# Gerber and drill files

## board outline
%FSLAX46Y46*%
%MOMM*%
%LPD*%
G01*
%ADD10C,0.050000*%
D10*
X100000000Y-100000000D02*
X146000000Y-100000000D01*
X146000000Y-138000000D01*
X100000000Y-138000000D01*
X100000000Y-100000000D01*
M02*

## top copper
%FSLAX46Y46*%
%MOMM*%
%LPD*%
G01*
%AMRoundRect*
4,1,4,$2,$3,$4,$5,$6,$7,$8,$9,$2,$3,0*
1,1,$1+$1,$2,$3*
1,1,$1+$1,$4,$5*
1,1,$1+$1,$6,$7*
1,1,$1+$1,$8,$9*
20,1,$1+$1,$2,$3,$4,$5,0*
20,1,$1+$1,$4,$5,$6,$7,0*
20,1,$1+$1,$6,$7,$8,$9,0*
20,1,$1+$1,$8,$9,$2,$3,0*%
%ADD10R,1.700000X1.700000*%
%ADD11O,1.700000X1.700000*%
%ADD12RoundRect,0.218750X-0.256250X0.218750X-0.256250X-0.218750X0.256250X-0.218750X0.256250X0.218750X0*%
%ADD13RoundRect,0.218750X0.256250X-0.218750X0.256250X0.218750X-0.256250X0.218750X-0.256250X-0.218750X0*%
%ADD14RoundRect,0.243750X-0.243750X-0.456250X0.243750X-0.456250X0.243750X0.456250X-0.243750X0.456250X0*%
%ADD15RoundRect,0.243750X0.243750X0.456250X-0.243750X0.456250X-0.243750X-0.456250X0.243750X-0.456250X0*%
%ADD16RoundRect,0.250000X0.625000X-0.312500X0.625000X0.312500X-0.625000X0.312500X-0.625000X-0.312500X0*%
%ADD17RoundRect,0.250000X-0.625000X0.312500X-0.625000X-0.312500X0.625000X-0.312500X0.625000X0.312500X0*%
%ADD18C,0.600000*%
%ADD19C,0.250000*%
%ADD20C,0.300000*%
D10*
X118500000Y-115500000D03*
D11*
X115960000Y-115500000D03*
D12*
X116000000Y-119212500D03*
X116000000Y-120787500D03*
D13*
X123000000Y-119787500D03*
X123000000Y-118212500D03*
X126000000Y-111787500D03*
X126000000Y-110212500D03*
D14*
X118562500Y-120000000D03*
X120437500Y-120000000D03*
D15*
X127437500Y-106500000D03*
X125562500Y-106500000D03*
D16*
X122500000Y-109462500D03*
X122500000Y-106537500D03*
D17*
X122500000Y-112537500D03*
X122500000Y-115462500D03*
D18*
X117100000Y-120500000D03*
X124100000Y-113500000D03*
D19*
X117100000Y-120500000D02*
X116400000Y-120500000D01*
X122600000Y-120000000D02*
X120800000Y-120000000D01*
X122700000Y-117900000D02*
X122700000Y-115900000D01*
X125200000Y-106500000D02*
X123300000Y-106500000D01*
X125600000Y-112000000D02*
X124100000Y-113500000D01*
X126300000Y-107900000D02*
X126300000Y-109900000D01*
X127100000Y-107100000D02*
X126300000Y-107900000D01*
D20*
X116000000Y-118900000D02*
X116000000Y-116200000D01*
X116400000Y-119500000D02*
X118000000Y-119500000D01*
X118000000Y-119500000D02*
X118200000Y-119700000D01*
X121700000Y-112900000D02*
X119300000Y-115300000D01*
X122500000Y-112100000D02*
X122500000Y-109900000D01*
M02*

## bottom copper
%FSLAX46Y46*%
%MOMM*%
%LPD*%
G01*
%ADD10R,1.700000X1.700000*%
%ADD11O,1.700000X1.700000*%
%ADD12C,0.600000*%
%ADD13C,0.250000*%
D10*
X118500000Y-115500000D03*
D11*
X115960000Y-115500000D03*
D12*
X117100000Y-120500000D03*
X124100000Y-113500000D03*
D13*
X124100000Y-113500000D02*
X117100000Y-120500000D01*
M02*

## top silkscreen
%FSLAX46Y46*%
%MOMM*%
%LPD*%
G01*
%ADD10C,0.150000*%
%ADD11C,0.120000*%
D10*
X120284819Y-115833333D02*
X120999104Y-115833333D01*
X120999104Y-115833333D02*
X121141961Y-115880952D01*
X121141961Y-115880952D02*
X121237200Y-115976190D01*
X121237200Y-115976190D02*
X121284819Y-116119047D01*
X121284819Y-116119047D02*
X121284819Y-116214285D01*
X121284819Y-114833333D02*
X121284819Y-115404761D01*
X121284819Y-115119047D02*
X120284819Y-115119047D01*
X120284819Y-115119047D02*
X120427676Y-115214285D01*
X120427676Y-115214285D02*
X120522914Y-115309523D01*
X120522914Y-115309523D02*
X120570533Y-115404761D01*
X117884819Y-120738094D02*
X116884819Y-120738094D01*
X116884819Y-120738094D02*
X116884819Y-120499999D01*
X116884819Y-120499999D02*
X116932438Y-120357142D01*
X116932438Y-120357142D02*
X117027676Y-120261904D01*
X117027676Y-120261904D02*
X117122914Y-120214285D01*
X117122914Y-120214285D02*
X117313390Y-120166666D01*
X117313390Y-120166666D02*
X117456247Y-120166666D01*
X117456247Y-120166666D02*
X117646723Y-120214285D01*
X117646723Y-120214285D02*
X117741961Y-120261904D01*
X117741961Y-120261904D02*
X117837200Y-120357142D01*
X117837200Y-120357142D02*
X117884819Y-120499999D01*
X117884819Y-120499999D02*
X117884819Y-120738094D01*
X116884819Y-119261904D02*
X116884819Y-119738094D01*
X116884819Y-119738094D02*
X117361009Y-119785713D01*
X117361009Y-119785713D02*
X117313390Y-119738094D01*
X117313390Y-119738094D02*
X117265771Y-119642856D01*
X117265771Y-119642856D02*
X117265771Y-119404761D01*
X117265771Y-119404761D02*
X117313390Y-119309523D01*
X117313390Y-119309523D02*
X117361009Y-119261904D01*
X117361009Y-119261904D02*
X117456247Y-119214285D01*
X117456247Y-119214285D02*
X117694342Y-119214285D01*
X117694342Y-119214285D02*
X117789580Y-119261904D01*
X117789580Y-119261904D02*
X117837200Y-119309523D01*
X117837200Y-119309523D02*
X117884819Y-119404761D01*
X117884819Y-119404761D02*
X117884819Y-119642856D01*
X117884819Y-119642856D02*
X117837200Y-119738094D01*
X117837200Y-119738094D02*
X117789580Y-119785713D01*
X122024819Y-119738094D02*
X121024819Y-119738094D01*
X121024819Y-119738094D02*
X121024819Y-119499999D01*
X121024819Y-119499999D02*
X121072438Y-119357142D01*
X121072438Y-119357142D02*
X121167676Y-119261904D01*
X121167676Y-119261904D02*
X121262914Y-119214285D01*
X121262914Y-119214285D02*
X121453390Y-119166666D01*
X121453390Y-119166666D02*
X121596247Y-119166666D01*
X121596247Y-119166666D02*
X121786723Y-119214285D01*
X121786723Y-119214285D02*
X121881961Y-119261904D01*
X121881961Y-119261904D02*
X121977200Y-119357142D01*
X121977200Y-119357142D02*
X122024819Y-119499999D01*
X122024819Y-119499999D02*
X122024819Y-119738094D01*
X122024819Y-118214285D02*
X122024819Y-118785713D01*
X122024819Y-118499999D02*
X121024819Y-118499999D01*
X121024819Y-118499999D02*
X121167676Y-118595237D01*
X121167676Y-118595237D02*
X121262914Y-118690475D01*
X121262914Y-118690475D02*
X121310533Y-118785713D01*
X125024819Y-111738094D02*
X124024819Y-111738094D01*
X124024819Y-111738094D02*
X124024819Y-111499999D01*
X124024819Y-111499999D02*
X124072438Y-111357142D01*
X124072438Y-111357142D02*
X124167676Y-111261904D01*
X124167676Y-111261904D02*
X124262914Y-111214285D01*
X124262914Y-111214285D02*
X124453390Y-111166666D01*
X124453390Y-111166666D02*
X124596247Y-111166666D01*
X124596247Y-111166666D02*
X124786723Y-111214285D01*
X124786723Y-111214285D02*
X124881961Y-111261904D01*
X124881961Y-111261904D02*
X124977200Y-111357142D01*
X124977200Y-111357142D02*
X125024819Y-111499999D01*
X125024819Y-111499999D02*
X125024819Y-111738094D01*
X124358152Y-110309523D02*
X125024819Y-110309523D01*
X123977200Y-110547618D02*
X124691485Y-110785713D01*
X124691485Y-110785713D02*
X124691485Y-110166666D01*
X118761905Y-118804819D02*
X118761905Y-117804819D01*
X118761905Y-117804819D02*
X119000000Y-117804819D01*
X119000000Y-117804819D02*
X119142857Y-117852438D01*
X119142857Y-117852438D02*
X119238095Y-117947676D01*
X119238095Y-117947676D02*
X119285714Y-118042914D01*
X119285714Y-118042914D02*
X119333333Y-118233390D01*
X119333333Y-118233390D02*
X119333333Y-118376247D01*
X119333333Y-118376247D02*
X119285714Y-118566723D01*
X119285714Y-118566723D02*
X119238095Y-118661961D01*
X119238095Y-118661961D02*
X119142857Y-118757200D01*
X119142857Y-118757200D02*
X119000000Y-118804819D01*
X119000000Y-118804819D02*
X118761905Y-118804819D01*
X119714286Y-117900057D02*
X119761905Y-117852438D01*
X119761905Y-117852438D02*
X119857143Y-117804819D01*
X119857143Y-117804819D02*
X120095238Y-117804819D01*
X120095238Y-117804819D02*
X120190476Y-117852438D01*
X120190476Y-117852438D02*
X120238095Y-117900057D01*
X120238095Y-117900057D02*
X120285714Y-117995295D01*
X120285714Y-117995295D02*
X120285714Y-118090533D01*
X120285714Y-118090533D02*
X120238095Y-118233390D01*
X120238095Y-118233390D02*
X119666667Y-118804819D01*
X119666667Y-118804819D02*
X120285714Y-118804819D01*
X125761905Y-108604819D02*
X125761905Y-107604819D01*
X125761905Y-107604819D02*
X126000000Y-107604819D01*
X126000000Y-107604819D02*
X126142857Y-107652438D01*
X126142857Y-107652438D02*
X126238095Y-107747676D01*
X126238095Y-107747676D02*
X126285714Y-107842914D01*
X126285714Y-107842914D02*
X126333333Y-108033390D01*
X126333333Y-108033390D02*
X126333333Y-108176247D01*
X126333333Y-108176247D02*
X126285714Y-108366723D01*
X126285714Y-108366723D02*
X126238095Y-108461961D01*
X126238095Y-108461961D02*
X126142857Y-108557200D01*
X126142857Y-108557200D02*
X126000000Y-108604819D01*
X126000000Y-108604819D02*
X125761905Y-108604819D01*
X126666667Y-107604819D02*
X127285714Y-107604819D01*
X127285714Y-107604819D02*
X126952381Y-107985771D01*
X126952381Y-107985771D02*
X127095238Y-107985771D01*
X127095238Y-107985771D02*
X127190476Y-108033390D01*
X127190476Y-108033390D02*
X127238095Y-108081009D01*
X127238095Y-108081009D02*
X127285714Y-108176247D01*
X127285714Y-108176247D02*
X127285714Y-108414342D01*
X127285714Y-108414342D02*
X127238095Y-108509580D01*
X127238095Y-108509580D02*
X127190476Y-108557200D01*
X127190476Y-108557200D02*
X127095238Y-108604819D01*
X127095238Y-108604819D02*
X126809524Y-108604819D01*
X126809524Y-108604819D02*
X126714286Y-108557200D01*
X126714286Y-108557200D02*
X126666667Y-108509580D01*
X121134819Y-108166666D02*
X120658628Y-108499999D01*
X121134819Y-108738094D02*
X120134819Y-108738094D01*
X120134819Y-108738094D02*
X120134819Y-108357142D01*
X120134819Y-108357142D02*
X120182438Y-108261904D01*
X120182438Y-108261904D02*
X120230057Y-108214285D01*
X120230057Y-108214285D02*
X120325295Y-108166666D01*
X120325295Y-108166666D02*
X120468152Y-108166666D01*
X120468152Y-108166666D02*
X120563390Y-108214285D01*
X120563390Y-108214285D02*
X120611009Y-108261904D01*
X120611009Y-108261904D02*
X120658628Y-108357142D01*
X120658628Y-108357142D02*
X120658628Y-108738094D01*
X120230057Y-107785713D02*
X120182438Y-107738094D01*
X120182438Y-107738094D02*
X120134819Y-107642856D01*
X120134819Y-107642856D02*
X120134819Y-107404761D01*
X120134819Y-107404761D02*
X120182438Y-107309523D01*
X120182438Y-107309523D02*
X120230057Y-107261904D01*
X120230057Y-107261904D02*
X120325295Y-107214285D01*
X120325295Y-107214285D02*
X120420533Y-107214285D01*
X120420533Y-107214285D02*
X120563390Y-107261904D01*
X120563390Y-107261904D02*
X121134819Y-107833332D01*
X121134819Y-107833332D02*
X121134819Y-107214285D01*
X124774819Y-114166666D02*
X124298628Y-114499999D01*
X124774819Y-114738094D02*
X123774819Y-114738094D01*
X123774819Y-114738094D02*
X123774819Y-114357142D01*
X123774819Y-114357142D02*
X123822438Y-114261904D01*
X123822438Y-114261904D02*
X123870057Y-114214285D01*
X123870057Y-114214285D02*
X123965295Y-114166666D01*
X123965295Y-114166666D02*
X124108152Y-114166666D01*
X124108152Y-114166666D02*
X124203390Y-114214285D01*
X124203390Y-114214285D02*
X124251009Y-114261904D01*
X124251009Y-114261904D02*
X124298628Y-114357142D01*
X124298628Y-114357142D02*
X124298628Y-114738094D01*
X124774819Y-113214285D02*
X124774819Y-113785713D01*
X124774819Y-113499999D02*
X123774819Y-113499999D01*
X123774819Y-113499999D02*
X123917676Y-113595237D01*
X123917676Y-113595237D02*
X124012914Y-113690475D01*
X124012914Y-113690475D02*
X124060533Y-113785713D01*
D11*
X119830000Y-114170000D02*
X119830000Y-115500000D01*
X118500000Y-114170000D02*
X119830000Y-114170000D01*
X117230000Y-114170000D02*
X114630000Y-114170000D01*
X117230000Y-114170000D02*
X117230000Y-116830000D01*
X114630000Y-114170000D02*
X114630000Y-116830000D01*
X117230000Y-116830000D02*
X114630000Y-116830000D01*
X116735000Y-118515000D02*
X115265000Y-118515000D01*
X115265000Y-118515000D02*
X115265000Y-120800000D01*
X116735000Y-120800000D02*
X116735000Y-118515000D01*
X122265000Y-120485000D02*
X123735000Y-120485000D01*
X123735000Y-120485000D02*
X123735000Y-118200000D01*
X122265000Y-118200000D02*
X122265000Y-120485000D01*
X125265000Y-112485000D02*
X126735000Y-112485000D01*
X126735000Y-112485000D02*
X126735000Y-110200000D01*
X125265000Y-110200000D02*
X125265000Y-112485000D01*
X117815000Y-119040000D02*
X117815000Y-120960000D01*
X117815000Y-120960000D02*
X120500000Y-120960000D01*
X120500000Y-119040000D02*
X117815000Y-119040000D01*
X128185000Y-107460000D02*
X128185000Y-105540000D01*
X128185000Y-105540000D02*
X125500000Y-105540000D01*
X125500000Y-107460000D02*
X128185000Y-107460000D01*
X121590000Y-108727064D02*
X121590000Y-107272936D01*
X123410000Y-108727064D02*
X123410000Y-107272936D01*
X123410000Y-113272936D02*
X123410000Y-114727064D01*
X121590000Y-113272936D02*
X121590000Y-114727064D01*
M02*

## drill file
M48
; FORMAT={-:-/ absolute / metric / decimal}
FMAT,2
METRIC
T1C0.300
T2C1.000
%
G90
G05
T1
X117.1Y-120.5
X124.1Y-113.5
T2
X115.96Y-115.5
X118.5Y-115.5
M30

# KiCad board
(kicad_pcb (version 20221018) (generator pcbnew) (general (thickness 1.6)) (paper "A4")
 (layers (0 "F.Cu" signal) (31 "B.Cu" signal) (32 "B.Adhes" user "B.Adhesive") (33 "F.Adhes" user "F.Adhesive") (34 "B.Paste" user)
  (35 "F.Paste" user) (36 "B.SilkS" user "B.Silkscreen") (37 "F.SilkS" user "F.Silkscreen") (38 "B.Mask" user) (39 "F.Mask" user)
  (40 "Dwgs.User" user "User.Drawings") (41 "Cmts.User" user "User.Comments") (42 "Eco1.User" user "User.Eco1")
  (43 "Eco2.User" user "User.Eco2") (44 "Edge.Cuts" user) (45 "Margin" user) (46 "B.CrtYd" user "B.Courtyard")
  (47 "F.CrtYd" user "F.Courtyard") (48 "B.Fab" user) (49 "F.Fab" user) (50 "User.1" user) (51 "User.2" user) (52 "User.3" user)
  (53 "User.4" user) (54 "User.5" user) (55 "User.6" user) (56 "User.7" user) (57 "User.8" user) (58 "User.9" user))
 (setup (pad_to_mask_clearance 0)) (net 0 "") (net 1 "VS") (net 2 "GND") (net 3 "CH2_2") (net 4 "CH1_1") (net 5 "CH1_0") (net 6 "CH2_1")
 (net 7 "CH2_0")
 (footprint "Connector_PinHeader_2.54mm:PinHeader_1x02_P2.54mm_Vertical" (layer "F.Cu") (at 118.5 115.5 -90)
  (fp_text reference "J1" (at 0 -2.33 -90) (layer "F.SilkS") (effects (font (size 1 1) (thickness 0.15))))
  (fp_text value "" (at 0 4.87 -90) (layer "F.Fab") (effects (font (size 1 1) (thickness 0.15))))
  (fp_line (start -1.33 -1.33) (end 0 -1.33) (stroke (width 0.12) (type solid)) (layer "F.SilkS"))
  (fp_line (start -1.33 0) (end -1.33 -1.33) (stroke (width 0.12) (type solid)) (layer "F.SilkS"))
  (fp_line (start -1.33 1.27) (end -1.33 3.87) (stroke (width 0.12) (type solid)) (layer "F.SilkS"))
  (fp_line (start -1.33 1.27) (end 1.33 1.27) (stroke (width 0.12) (type solid)) (layer "F.SilkS"))
  (fp_line (start -1.33 3.87) (end 1.33 3.87) (stroke (width 0.12) (type solid)) (layer "F.SilkS"))
  (fp_line (start 1.33 1.27) (end 1.33 3.87) (stroke (width 0.12) (type solid)) (layer "F.SilkS"))
  (pad "1" thru_hole rect (at 0 0 270) (size 1.7 1.7) (drill 1) (layers "*.Cu" "*.Mask") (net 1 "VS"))
  (pad "2" thru_hole oval (at 0 2.54 270) (size 1.7 1.7) (drill 1) (layers "*.Cu" "*.Mask") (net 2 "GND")))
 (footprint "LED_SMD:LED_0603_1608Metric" (layer "F.Cu") (at 116 120 -90)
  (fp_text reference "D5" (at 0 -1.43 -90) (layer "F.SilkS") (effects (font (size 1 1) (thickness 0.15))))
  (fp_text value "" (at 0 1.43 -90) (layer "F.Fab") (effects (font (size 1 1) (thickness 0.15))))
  (fp_line (start -1.485 -0.735) (end -1.485 0.735) (stroke (width 0.12) (type solid)) (layer "F.SilkS"))
  (fp_line (start -1.485 0.735) (end 0.8 0.735) (stroke (width 0.12) (type solid)) (layer "F.SilkS"))
  (fp_line (start 0.8 -0.735) (end -1.485 -0.735) (stroke (width 0.12) (type solid)) (layer "F.SilkS"))
  (pad "1" smd roundrect (at -0.7875 0 270) (size 0.875 0.95) (layers "F.Cu" "F.Paste" "F.Mask") (roundrect_rratio 0.25) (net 2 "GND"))
  (pad "2" smd roundrect (at 0.7875 0 270) (size 0.875 0.95) (layers "F.Cu" "F.Paste" "F.Mask") (roundrect_rratio 0.25) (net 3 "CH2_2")))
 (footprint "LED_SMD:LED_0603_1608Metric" (layer "F.Cu") (at 123 119 90)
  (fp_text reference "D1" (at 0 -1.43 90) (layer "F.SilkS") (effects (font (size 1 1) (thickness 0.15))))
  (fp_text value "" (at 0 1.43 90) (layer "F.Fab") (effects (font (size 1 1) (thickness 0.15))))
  (fp_line (start -1.485 -0.735) (end -1.485 0.735) (stroke (width 0.12) (type solid)) (layer "F.SilkS"))
  (fp_line (start -1.485 0.735) (end 0.8 0.735) (stroke (width 0.12) (type solid)) (layer "F.SilkS"))
  (fp_line (start 0.8 -0.735) (end -1.485 -0.735) (stroke (width 0.12) (type solid)) (layer "F.SilkS"))
  (pad "1" smd roundrect (at -0.7875 0 90) (size 0.875 0.95) (layers "F.Cu" "F.Paste" "F.Mask") (roundrect_rratio 0.25) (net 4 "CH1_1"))
  (pad "2" smd roundrect (at 0.7875 0 90) (size 0.875 0.95) (layers "F.Cu" "F.Paste" "F.Mask") (roundrect_rratio 0.25) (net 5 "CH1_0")))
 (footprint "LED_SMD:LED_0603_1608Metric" (layer "F.Cu") (at 126 111 90)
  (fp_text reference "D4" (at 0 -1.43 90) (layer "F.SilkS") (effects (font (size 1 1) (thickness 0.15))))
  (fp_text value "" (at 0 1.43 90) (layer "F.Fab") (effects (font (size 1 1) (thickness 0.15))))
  (fp_line (start -1.485 -0.735) (end -1.485 0.735) (stroke (width 0.12) (type solid)) (layer "F.SilkS"))
  (fp_line (start -1.485 0.735) (end 0.8 0.735) (stroke (width 0.12) (type solid)) (layer "F.SilkS"))
  (fp_line (start 0.8 -0.735) (end -1.485 -0.735) (stroke (width 0.12) (type solid)) (layer "F.SilkS"))
  (pad "1" smd roundrect (at -0.7875 0 90) (size 0.875 0.95) (layers "F.Cu" "F.Paste" "F.Mask") (roundrect_rratio 0.25) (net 3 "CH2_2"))
  (pad "2" smd roundrect (at 0.7875 0 90) (size 0.875 0.95) (layers "F.Cu" "F.Paste" "F.Mask") (roundrect_rratio 0.25) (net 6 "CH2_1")))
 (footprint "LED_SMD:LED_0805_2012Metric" (layer "F.Cu") (at 119.5 120)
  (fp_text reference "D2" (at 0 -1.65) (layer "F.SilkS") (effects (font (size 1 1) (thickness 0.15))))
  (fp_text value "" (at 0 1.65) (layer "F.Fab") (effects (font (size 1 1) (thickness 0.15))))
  (fp_line (start -1.685 -0.96) (end -1.685 0.96) (stroke (width 0.12) (type solid)) (layer "F.SilkS"))
  (fp_line (start -1.685 0.96) (end 1 0.96) (stroke (width 0.12) (type solid)) (layer "F.SilkS"))
  (fp_line (start 1 -0.96) (end -1.685 -0.96) (stroke (width 0.12) (type solid)) (layer "F.SilkS"))
  (pad "1" smd roundrect (at -0.9375 0) (size 0.975 1.4) (layers "F.Cu" "F.Paste" "F.Mask") (roundrect_rratio 0.25) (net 2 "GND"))
  (pad "2" smd roundrect (at 0.9375 0) (size 0.975 1.4) (layers "F.Cu" "F.Paste" "F.Mask") (roundrect_rratio 0.25) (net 4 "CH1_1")))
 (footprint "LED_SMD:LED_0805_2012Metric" (layer "F.Cu") (at 126.5 106.5 180)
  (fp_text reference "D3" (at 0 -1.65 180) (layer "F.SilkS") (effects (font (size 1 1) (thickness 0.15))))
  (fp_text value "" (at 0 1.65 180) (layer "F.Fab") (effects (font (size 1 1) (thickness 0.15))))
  (fp_line (start -1.685 -0.96) (end -1.685 0.96) (stroke (width 0.12) (type solid)) (layer "F.SilkS"))
  (fp_line (start -1.685 0.96) (end 1 0.96) (stroke (width 0.12) (type solid)) (layer "F.SilkS"))
  (fp_line (start 1 -0.96) (end -1.685 -0.96) (stroke (width 0.12) (type solid)) (layer "F.SilkS"))
  (pad "1" smd roundrect (at -0.9375 0 180) (size 0.975 1.4) (layers "F.Cu" "F.Paste" "F.Mask") (roundrect_rratio 0.25) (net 6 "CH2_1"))
  (pad "2" smd roundrect (at 0.9375 0 180) (size 0.975 1.4) (layers "F.Cu" "F.Paste" "F.Mask") (roundrect_rratio 0.25) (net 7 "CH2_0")))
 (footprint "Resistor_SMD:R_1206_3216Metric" (layer "F.Cu") (at 122.5 108 90)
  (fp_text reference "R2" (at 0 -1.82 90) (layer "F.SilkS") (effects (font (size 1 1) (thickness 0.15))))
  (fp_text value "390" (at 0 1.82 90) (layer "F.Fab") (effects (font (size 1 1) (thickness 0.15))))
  (fp_line (start -0.727064 -0.91) (end 0.727064 -0.91) (stroke (width 0.12) (type solid)) (layer "F.SilkS"))
  (fp_line (start -0.727064 0.91) (end 0.727064 0.91) (stroke (width 0.12) (type solid)) (layer "F.SilkS"))
  (pad "1" smd roundrect (at -1.4625 0 90) (size 1.125 1.75) (layers "F.Cu" "F.Paste" "F.Mask") (roundrect_rratio 0.222222) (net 1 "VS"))
  (pad "2" smd roundrect (at 1.4625 0 90) (size 1.125 1.75) (layers "F.Cu" "F.Paste" "F.Mask") (roundrect_rratio 0.222222) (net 7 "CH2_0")))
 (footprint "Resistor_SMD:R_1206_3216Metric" (layer "F.Cu") (at 122.5 114 -90)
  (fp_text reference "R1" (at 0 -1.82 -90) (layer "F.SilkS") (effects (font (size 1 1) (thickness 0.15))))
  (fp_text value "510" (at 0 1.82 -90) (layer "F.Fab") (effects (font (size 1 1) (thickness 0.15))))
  (fp_line (start -0.727064 -0.91) (end 0.727064 -0.91) (stroke (width 0.12) (type solid)) (layer "F.SilkS"))
  (fp_line (start -0.727064 0.91) (end 0.727064 0.91) (stroke (width 0.12) (type solid)) (layer "F.SilkS"))
  (pad "1" smd roundrect (at -1.4625 0 270) (size 1.125 1.75) (layers "F.Cu" "F.Paste" "F.Mask") (roundrect_rratio 0.222222) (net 1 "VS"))
  (pad "2" smd roundrect (at 1.4625 0 270) (size 1.125 1.75) (layers "F.Cu" "F.Paste" "F.Mask") (roundrect_rratio 0.222222) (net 5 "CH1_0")))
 (gr_rect (start 100 100) (end 146 138) (stroke (width 0.05) (type default)) (fill none) (layer "Edge.Cuts"))
 (segment (start 117.1 120.5) (end 116.4 120.5) (width 0.25) (layer "F.Cu") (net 3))
 (segment (start 122.6 120) (end 120.8 120) (width 0.25) (layer "F.Cu") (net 4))
 (segment (start 122.7 117.9) (end 122.7 115.9) (width 0.25) (layer "F.Cu") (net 5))
 (segment (start 125.2 106.5) (end 123.3 106.5) (width 0.25) (layer "F.Cu") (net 7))
 (segment (start 125.6 112) (end 124.1 113.5) (width 0.25) (layer "F.Cu") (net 3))
 (segment (start 126.3 107.9) (end 126.3 109.9) (width 0.25) (layer "F.Cu") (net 6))
 (segment (start 127.1 107.1) (end 126.3 107.9) (width 0.25) (layer "F.Cu") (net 6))
 (via (at 117.1 120.5) (size 0.6) (drill 0.3) (layers "F.Cu" "B.Cu") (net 3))
 (via (at 124.1 113.5) (size 0.6) (drill 0.3) (layers "F.Cu" "B.Cu") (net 3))
 (segment (start 116 118.9) (end 116 116.2) (width 0.3) (layer "F.Cu") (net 2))
 (segment (start 116.4 119.5) (end 118 119.5) (width 0.3) (layer "F.Cu") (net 2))
 (segment (start 118 119.5) (end 118.2 119.7) (width 0.3) (layer "F.Cu") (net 2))
 (segment (start 121.7 112.9) (end 119.3 115.3) (width 0.3) (layer "F.Cu") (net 1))
 (segment (start 122.5 112.1) (end 122.5 109.9) (width 0.3) (layer "F.Cu") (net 1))
 (segment (start 124.1 113.5) (end 117.1 120.5) (width 0.25) (layer "B.Cu") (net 3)))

